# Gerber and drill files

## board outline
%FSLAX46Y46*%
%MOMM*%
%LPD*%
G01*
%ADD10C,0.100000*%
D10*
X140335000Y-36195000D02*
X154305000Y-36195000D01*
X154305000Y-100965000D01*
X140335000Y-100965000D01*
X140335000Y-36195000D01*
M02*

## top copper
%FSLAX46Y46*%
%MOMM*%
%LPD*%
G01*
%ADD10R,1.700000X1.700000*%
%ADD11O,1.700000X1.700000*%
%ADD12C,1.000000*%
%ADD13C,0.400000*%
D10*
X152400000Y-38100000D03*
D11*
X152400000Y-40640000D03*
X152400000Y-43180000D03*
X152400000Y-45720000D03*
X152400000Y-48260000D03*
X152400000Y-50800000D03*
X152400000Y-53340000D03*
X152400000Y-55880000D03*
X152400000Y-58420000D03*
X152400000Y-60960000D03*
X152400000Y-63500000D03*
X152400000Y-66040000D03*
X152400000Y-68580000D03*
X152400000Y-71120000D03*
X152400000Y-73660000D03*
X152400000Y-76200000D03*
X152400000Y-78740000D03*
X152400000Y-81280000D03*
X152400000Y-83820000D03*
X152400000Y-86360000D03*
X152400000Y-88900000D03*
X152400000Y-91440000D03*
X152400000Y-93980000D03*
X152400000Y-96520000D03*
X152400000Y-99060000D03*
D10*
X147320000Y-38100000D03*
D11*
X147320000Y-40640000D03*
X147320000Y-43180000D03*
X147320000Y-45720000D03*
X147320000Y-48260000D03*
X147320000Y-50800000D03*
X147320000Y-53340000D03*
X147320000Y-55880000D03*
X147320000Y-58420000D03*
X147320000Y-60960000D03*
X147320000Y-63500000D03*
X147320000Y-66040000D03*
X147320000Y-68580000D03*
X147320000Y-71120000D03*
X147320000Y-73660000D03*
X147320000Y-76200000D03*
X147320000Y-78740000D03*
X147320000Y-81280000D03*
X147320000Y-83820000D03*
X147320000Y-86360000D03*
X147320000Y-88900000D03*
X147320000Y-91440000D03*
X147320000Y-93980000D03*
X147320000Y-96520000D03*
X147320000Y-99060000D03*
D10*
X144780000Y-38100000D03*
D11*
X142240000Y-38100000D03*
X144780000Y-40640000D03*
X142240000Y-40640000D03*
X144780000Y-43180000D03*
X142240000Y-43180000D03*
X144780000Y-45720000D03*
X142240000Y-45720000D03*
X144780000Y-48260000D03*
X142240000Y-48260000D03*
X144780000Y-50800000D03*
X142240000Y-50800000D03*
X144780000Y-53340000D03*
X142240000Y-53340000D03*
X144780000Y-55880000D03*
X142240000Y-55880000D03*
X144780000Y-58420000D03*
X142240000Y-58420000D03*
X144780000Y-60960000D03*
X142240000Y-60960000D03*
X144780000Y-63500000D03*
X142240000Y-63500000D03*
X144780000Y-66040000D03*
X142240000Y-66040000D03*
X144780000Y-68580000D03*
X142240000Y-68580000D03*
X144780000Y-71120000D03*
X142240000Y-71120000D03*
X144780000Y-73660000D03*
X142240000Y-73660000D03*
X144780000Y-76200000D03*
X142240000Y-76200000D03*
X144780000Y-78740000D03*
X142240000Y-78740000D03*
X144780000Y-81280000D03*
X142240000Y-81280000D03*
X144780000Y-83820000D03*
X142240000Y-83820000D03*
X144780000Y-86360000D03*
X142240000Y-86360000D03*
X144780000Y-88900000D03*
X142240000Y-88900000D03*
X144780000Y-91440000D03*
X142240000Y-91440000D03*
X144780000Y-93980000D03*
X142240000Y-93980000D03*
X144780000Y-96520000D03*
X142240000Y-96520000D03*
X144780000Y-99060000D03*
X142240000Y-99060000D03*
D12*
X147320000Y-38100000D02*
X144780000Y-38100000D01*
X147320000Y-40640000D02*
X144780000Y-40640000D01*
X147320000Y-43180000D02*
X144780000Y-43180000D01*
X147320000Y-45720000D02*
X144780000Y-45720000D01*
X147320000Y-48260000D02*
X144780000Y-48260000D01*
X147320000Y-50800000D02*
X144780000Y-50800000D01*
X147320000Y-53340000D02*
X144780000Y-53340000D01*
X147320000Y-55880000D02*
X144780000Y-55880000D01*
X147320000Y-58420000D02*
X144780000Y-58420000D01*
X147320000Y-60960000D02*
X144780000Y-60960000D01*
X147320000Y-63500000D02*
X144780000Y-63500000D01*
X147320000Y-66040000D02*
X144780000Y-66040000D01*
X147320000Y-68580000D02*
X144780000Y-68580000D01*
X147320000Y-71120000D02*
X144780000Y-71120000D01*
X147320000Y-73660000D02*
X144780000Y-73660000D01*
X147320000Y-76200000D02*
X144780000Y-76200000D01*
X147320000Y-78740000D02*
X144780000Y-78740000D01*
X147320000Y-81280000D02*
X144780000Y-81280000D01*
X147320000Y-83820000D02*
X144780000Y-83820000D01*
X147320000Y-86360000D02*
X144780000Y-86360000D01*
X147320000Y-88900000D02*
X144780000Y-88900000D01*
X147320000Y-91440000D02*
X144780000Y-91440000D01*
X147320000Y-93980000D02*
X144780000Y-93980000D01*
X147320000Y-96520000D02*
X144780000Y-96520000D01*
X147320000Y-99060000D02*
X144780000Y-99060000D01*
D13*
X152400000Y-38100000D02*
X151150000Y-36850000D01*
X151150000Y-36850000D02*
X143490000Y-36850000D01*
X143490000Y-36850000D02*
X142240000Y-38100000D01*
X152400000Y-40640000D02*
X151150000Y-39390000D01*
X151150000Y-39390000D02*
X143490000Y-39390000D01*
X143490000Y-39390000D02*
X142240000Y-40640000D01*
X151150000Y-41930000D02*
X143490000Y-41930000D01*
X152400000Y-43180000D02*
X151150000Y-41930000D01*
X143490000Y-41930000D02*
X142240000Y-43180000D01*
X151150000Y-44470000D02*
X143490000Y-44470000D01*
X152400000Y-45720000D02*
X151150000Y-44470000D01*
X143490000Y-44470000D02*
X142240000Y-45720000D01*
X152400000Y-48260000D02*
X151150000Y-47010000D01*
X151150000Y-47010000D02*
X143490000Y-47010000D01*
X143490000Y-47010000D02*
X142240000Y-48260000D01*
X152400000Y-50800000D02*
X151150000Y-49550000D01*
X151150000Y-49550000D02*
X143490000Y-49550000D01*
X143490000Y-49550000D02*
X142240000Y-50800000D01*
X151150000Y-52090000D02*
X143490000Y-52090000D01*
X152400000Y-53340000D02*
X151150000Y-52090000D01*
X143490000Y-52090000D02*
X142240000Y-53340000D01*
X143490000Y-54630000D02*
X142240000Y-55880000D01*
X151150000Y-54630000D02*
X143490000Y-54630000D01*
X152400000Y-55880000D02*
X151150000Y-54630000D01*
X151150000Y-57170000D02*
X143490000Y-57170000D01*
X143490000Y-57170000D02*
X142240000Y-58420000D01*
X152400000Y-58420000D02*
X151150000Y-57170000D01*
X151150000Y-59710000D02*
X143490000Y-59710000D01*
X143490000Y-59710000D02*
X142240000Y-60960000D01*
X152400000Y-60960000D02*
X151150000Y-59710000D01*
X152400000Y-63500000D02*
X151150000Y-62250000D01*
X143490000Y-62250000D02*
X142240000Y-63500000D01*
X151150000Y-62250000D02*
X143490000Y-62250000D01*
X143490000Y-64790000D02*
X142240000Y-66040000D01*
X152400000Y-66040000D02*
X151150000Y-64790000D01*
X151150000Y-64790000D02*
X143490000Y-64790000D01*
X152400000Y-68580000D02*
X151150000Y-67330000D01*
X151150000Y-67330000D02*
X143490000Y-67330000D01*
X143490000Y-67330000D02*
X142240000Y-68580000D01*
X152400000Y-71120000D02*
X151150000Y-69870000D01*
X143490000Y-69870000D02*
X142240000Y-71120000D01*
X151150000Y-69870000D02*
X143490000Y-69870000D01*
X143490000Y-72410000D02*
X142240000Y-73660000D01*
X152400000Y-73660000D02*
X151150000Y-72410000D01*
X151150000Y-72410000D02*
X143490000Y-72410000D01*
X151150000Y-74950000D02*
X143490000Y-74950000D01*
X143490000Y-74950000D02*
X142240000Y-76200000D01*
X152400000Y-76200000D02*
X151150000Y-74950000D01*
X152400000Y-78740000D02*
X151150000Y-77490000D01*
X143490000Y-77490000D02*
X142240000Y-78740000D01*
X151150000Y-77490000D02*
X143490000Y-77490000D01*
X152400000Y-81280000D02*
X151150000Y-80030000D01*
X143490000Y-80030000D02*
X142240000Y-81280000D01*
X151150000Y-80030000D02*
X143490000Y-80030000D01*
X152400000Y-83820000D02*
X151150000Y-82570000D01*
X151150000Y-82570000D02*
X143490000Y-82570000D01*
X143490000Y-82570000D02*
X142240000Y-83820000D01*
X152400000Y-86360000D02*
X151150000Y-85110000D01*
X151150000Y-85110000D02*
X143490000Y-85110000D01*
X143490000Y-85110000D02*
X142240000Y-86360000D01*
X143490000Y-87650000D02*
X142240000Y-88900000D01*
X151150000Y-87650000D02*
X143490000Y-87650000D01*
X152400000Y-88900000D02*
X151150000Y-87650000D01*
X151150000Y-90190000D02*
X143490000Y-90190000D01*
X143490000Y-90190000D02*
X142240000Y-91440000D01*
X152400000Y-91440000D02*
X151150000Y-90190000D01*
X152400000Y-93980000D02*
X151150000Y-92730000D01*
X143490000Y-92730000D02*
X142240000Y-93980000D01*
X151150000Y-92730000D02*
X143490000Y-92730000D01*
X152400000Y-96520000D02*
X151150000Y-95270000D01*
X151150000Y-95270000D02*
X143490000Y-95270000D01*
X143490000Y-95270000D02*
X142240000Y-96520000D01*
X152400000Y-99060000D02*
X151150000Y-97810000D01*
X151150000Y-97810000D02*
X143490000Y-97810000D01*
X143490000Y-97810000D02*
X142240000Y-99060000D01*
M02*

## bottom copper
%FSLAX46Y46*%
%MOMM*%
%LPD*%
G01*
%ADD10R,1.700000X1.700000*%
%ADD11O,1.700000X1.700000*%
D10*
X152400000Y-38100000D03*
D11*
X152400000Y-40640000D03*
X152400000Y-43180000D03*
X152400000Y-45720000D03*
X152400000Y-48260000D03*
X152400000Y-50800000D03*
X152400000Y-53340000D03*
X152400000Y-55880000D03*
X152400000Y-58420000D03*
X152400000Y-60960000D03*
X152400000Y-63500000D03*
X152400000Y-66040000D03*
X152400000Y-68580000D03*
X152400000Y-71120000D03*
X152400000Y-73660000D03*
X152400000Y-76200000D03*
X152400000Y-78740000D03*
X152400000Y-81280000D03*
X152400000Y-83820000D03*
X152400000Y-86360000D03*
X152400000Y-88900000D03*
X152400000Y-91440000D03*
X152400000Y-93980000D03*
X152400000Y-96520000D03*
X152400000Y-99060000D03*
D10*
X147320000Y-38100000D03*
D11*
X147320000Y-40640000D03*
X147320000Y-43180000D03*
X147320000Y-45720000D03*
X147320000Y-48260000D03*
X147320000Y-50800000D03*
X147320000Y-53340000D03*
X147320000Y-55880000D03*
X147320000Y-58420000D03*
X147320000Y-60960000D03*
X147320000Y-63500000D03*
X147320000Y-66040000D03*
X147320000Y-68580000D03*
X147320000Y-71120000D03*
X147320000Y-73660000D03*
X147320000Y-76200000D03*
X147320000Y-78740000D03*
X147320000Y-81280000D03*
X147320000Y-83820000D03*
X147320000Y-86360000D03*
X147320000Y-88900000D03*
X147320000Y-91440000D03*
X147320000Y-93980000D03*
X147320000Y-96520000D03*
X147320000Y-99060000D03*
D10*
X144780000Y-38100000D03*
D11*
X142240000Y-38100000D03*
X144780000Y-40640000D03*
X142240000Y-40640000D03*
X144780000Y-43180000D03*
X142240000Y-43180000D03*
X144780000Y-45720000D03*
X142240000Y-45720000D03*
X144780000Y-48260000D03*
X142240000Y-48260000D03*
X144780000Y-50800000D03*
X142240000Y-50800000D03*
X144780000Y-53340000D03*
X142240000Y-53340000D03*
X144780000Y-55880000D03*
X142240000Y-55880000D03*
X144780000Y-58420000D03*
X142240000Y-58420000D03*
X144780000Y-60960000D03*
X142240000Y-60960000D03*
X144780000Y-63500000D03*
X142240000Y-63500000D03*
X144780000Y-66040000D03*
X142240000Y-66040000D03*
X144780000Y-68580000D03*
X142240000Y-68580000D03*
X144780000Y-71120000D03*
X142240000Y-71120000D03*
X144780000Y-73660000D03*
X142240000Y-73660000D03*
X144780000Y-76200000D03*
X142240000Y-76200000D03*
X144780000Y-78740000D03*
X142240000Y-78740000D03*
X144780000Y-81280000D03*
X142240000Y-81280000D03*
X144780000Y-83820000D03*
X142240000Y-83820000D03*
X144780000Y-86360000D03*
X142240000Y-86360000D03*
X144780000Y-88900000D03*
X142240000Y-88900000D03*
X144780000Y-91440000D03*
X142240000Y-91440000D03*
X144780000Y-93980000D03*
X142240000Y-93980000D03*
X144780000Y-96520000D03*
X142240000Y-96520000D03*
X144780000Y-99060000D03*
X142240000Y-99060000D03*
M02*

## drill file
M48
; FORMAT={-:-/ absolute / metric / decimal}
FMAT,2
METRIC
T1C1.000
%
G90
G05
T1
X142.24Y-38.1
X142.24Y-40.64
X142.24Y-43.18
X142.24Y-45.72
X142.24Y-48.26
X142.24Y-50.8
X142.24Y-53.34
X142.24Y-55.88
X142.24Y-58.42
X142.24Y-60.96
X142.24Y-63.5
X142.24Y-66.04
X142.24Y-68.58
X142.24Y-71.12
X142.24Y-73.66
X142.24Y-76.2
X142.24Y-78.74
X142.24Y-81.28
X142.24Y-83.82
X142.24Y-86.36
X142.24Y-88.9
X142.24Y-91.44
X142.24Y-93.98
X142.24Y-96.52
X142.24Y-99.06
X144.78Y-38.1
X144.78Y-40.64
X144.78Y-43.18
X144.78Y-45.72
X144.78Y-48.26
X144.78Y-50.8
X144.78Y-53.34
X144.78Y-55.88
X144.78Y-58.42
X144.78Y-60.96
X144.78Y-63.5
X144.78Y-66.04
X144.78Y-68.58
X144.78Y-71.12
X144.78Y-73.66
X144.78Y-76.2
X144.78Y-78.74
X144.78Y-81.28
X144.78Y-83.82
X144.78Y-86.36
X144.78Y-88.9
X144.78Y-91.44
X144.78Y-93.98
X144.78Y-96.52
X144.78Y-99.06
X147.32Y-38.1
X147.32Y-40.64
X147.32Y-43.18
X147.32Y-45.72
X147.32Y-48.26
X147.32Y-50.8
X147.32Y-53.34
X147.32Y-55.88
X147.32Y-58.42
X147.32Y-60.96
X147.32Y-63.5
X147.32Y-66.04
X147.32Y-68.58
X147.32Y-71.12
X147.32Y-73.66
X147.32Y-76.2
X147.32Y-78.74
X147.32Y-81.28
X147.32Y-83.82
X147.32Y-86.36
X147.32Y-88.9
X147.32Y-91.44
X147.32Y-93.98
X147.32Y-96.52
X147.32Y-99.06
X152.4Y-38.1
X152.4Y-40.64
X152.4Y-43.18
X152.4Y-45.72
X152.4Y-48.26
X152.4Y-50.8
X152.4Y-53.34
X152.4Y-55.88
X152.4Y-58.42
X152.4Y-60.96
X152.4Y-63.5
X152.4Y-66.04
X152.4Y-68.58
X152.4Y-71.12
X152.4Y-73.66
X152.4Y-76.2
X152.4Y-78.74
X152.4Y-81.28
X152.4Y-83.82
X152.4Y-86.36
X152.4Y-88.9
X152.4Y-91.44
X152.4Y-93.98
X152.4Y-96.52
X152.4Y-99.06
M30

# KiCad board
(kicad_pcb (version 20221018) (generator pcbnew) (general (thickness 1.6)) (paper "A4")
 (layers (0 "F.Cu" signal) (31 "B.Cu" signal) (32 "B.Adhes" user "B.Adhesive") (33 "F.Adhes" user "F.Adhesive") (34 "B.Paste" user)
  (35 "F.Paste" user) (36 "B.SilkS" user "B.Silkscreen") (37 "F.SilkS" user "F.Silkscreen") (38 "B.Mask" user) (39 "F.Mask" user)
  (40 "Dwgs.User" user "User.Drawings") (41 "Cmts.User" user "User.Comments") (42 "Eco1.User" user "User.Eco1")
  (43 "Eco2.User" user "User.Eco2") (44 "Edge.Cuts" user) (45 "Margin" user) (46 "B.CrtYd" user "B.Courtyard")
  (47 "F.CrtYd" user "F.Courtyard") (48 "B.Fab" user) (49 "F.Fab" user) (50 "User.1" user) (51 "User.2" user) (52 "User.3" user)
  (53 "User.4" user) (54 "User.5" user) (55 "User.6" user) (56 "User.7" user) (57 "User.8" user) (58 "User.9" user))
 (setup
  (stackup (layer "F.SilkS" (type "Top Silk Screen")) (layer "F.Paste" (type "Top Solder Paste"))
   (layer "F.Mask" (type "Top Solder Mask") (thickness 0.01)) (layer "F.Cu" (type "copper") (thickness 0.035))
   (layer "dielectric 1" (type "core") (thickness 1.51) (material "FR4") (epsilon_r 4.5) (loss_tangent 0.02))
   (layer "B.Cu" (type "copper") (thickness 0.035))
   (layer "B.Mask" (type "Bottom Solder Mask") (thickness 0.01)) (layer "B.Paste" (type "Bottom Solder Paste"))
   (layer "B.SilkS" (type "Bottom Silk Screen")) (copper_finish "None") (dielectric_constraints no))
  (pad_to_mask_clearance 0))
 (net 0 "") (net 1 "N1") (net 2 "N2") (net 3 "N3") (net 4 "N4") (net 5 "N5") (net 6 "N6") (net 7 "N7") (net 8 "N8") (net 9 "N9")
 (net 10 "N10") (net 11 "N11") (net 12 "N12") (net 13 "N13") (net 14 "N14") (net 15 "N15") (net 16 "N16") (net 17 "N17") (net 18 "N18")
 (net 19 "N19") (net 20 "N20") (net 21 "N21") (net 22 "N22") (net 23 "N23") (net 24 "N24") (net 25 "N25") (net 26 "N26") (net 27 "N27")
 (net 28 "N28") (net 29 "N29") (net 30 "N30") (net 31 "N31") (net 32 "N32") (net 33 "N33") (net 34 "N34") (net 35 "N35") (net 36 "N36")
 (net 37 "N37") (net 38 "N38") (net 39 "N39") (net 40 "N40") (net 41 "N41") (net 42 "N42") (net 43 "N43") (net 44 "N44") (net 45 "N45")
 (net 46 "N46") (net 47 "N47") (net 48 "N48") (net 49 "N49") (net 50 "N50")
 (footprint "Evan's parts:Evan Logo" (layer "F.Cu") (at 149.86 49.53 90)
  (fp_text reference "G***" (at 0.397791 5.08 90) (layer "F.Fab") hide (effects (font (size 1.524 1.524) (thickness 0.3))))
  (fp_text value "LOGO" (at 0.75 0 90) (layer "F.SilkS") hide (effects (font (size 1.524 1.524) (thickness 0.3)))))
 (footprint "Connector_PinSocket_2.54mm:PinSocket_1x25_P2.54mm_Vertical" (layer "F.Cu") (at 152.4 38.1)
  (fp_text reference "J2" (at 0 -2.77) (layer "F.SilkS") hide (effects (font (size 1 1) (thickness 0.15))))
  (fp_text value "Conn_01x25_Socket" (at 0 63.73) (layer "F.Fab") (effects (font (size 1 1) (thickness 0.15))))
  (pad "1" thru_hole rect (at 0 0) (size 1.7 1.7) (drill 1) (layers "*.Cu" "*.Mask") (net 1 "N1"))
  (pad "2" thru_hole oval (at 0 2.54) (size 1.7 1.7) (drill 1) (layers "*.Cu" "*.Mask") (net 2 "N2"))
  (pad "3" thru_hole oval (at 0 5.08) (size 1.7 1.7) (drill 1) (layers "*.Cu" "*.Mask") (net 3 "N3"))
  (pad "4" thru_hole oval (at 0 7.62) (size 1.7 1.7) (drill 1) (layers "*.Cu" "*.Mask") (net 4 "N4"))
  (pad "5" thru_hole oval (at 0 10.16) (size 1.7 1.7) (drill 1) (layers "*.Cu" "*.Mask") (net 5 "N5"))
  (pad "6" thru_hole oval (at 0 12.7) (size 1.7 1.7) (drill 1) (layers "*.Cu" "*.Mask") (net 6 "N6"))
  (pad "7" thru_hole oval (at 0 15.24) (size 1.7 1.7) (drill 1) (layers "*.Cu" "*.Mask") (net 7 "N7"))
  (pad "8" thru_hole oval (at 0 17.78) (size 1.7 1.7) (drill 1) (layers "*.Cu" "*.Mask") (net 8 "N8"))
  (pad "9" thru_hole oval (at 0 20.32) (size 1.7 1.7) (drill 1) (layers "*.Cu" "*.Mask") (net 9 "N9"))
  (pad "10" thru_hole oval (at 0 22.86) (size 1.7 1.7) (drill 1) (layers "*.Cu" "*.Mask") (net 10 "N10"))
  (pad "11" thru_hole oval (at 0 25.4) (size 1.7 1.7) (drill 1) (layers "*.Cu" "*.Mask") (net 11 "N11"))
  (pad "12" thru_hole oval (at 0 27.94) (size 1.7 1.7) (drill 1) (layers "*.Cu" "*.Mask") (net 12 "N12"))
  (pad "13" thru_hole oval (at 0 30.48) (size 1.7 1.7) (drill 1) (layers "*.Cu" "*.Mask") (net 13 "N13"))
  (pad "14" thru_hole oval (at 0 33.02) (size 1.7 1.7) (drill 1) (layers "*.Cu" "*.Mask") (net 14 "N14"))
  (pad "15" thru_hole oval (at 0 35.56) (size 1.7 1.7) (drill 1) (layers "*.Cu" "*.Mask") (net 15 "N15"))
  (pad "16" thru_hole oval (at 0 38.1) (size 1.7 1.7) (drill 1) (layers "*.Cu" "*.Mask") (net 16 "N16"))
  (pad "17" thru_hole oval (at 0 40.64) (size 1.7 1.7) (drill 1) (layers "*.Cu" "*.Mask") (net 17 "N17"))
  (pad "18" thru_hole oval (at 0 43.18) (size 1.7 1.7) (drill 1) (layers "*.Cu" "*.Mask") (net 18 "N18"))
  (pad "19" thru_hole oval (at 0 45.72) (size 1.7 1.7) (drill 1) (layers "*.Cu" "*.Mask") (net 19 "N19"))
  (pad "20" thru_hole oval (at 0 48.26) (size 1.7 1.7) (drill 1) (layers "*.Cu" "*.Mask") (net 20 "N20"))
  (pad "21" thru_hole oval (at 0 50.8) (size 1.7 1.7) (drill 1) (layers "*.Cu" "*.Mask") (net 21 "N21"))
  (pad "22" thru_hole oval (at 0 53.34) (size 1.7 1.7) (drill 1) (layers "*.Cu" "*.Mask") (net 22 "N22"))
  (pad "23" thru_hole oval (at 0 55.88) (size 1.7 1.7) (drill 1) (layers "*.Cu" "*.Mask") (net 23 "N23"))
  (pad "24" thru_hole oval (at 0 58.42) (size 1.7 1.7) (drill 1) (layers "*.Cu" "*.Mask") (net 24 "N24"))
  (pad "25" thru_hole oval (at 0 60.96) (size 1.7 1.7) (drill 1) (layers "*.Cu" "*.Mask") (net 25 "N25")))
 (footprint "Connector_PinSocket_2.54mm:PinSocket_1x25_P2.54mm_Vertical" (layer "F.Cu") (at 147.32 38.1)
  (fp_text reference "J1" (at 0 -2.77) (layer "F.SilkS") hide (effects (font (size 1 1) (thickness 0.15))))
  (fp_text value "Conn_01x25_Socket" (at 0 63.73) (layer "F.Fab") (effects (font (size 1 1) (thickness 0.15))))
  (pad "1" thru_hole rect (at 0 0) (size 1.7 1.7) (drill 1) (layers "*.Cu" "*.Mask") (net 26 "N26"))
  (pad "2" thru_hole oval (at 0 2.54) (size 1.7 1.7) (drill 1) (layers "*.Cu" "*.Mask") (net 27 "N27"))
  (pad "3" thru_hole oval (at 0 5.08) (size 1.7 1.7) (drill 1) (layers "*.Cu" "*.Mask") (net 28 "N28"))
  (pad "4" thru_hole oval (at 0 7.62) (size 1.7 1.7) (drill 1) (layers "*.Cu" "*.Mask") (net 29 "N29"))
  (pad "5" thru_hole oval (at 0 10.16) (size 1.7 1.7) (drill 1) (layers "*.Cu" "*.Mask") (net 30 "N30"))
  (pad "6" thru_hole oval (at 0 12.7) (size 1.7 1.7) (drill 1) (layers "*.Cu" "*.Mask") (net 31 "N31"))
  (pad "7" thru_hole oval (at 0 15.24) (size 1.7 1.7) (drill 1) (layers "*.Cu" "*.Mask") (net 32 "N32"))
  (pad "8" thru_hole oval (at 0 17.78) (size 1.7 1.7) (drill 1) (layers "*.Cu" "*.Mask") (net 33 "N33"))
  (pad "9" thru_hole oval (at 0 20.32) (size 1.7 1.7) (drill 1) (layers "*.Cu" "*.Mask") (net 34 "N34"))
  (pad "10" thru_hole oval (at 0 22.86) (size 1.7 1.7) (drill 1) (layers "*.Cu" "*.Mask") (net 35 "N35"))
  (pad "11" thru_hole oval (at 0 25.4) (size 1.7 1.7) (drill 1) (layers "*.Cu" "*.Mask") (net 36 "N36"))
  (pad "12" thru_hole oval (at 0 27.94) (size 1.7 1.7) (drill 1) (layers "*.Cu" "*.Mask") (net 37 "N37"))
  (pad "13" thru_hole oval (at 0 30.48) (size 1.7 1.7) (drill 1) (layers "*.Cu" "*.Mask") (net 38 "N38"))
  (pad "14" thru_hole oval (at 0 33.02) (size 1.7 1.7) (drill 1) (layers "*.Cu" "*.Mask") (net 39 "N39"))
  (pad "15" thru_hole oval (at 0 35.56) (size 1.7 1.7) (drill 1) (layers "*.Cu" "*.Mask") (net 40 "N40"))
  (pad "16" thru_hole oval (at 0 38.1) (size 1.7 1.7) (drill 1) (layers "*.Cu" "*.Mask") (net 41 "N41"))
  (pad "17" thru_hole oval (at 0 40.64) (size 1.7 1.7) (drill 1) (layers "*.Cu" "*.Mask") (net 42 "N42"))
  (pad "18" thru_hole oval (at 0 43.18) (size 1.7 1.7) (drill 1) (layers "*.Cu" "*.Mask") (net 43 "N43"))
  (pad "19" thru_hole oval (at 0 45.72) (size 1.7 1.7) (drill 1) (layers "*.Cu" "*.Mask") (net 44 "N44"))
  (pad "20" thru_hole oval (at 0 48.26) (size 1.7 1.7) (drill 1) (layers "*.Cu" "*.Mask") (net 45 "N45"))
  (pad "21" thru_hole oval (at 0 50.8) (size 1.7 1.7) (drill 1) (layers "*.Cu" "*.Mask") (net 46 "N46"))
  (pad "22" thru_hole oval (at 0 53.34) (size 1.7 1.7) (drill 1) (layers "*.Cu" "*.Mask") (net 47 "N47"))
  (pad "23" thru_hole oval (at 0 55.88) (size 1.7 1.7) (drill 1) (layers "*.Cu" "*.Mask") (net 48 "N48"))
  (pad "24" thru_hole oval (at 0 58.42) (size 1.7 1.7) (drill 1) (layers "*.Cu" "*.Mask") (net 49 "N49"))
  (pad "25" thru_hole oval (at 0 60.96) (size 1.7 1.7) (drill 1) (layers "*.Cu" "*.Mask") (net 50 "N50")))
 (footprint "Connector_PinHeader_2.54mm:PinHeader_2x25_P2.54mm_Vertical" (layer "B.Cu") (at 144.78 38.1 180)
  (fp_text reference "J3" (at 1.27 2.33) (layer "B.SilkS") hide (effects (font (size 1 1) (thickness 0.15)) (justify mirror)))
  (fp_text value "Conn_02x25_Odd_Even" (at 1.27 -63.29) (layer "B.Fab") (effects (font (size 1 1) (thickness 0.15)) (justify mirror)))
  (pad "1" thru_hole rect (at 0 0 180) (size 1.7 1.7) (drill 1) (layers "*.Cu" "*.Mask") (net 26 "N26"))
  (pad "2" thru_hole oval (at 2.54 0 180) (size 1.7 1.7) (drill 1) (layers "*.Cu" "*.Mask") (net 1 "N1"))
  (pad "3" thru_hole oval (at 0 -2.54 180) (size 1.7 1.7) (drill 1) (layers "*.Cu" "*.Mask") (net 27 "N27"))
  (pad "4" thru_hole oval (at 2.54 -2.54 180) (size 1.7 1.7) (drill 1) (layers "*.Cu" "*.Mask") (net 2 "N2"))
  (pad "5" thru_hole oval (at 0 -5.08 180) (size 1.7 1.7) (drill 1) (layers "*.Cu" "*.Mask") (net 28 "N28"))
  (pad "6" thru_hole oval (at 2.54 -5.08 180) (size 1.7 1.7) (drill 1) (layers "*.Cu" "*.Mask") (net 3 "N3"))
  (pad "7" thru_hole oval (at 0 -7.62 180) (size 1.7 1.7) (drill 1) (layers "*.Cu" "*.Mask") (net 29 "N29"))
  (pad "8" thru_hole oval (at 2.54 -7.62 180) (size 1.7 1.7) (drill 1) (layers "*.Cu" "*.Mask") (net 4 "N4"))
  (pad "9" thru_hole oval (at 0 -10.16 180) (size 1.7 1.7) (drill 1) (layers "*.Cu" "*.Mask") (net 30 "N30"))
  (pad "10" thru_hole oval (at 2.54 -10.16 180) (size 1.7 1.7) (drill 1) (layers "*.Cu" "*.Mask") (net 5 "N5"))
  (pad "11" thru_hole oval (at 0 -12.7 180) (size 1.7 1.7) (drill 1) (layers "*.Cu" "*.Mask") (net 31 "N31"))
  (pad "12" thru_hole oval (at 2.54 -12.7 180) (size 1.7 1.7) (drill 1) (layers "*.Cu" "*.Mask") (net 6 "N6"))
  (pad "13" thru_hole oval (at 0 -15.24 180) (size 1.7 1.7) (drill 1) (layers "*.Cu" "*.Mask") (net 32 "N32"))
  (pad "14" thru_hole oval (at 2.54 -15.24 180) (size 1.7 1.7) (drill 1) (layers "*.Cu" "*.Mask") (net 7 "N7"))
  (pad "15" thru_hole oval (at 0 -17.78 180) (size 1.7 1.7) (drill 1) (layers "*.Cu" "*.Mask") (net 33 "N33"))
  (pad "16" thru_hole oval (at 2.54 -17.78 180) (size 1.7 1.7) (drill 1) (layers "*.Cu" "*.Mask") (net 8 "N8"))
  (pad "17" thru_hole oval (at 0 -20.32 180) (size 1.7 1.7) (drill 1) (layers "*.Cu" "*.Mask") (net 34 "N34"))
  (pad "18" thru_hole oval (at 2.54 -20.32 180) (size 1.7 1.7) (drill 1) (layers "*.Cu" "*.Mask") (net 9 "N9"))
  (pad "19" thru_hole oval (at 0 -22.86 180) (size 1.7 1.7) (drill 1) (layers "*.Cu" "*.Mask") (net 35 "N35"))
  (pad "20" thru_hole oval (at 2.54 -22.86 180) (size 1.7 1.7) (drill 1) (layers "*.Cu" "*.Mask") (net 10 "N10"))
  (pad "21" thru_hole oval (at 0 -25.4 180) (size 1.7 1.7) (drill 1) (layers "*.Cu" "*.Mask") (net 36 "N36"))
  (pad "22" thru_hole oval (at 2.54 -25.4 180) (size 1.7 1.7) (drill 1) (layers "*.Cu" "*.Mask") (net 11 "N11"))
  (pad "23" thru_hole oval (at 0 -27.94 180) (size 1.7 1.7) (drill 1) (layers "*.Cu" "*.Mask") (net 37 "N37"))
  (pad "24" thru_hole oval (at 2.54 -27.94 180) (size 1.7 1.7) (drill 1) (layers "*.Cu" "*.Mask") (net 12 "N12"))
  (pad "25" thru_hole oval (at 0 -30.48 180) (size 1.7 1.7) (drill 1) (layers "*.Cu" "*.Mask") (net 38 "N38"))
  (pad "26" thru_hole oval (at 2.54 -30.48 180) (size 1.7 1.7) (drill 1) (layers "*.Cu" "*.Mask") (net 13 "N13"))
  (pad "27" thru_hole oval (at 0 -33.02 180) (size 1.7 1.7) (drill 1) (layers "*.Cu" "*.Mask") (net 39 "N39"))
  (pad "28" thru_hole oval (at 2.54 -33.02 180) (size 1.7 1.7) (drill 1) (layers "*.Cu" "*.Mask") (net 14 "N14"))
  (pad "29" thru_hole oval (at 0 -35.56 180) (size 1.7 1.7) (drill 1) (layers "*.Cu" "*.Mask") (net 40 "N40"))
  (pad "30" thru_hole oval (at 2.54 -35.56 180) (size 1.7 1.7) (drill 1) (layers "*.Cu" "*.Mask") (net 15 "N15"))
  (pad "31" thru_hole oval (at 0 -38.1 180) (size 1.7 1.7) (drill 1) (layers "*.Cu" "*.Mask") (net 41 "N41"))
  (pad "32" thru_hole oval (at 2.54 -38.1 180) (size 1.7 1.7) (drill 1) (layers "*.Cu" "*.Mask") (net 16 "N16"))
  (pad "33" thru_hole oval (at 0 -40.64 180) (size 1.7 1.7) (drill 1) (layers "*.Cu" "*.Mask") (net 42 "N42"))
  (pad "34" thru_hole oval (at 2.54 -40.64 180) (size 1.7 1.7) (drill 1) (layers "*.Cu" "*.Mask") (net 17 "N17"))
  (pad "35" thru_hole oval (at 0 -43.18 180) (size 1.7 1.7) (drill 1) (layers "*.Cu" "*.Mask") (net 43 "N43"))
  (pad "36" thru_hole oval (at 2.54 -43.18 180) (size 1.7 1.7) (drill 1) (layers "*.Cu" "*.Mask") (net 18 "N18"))
  (pad "37" thru_hole oval (at 0 -45.72 180) (size 1.7 1.7) (drill 1) (layers "*.Cu" "*.Mask") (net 44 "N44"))
  (pad "38" thru_hole oval (at 2.54 -45.72 180) (size 1.7 1.7) (drill 1) (layers "*.Cu" "*.Mask") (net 19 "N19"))
  (pad "39" thru_hole oval (at 0 -48.26 180) (size 1.7 1.7) (drill 1) (layers "*.Cu" "*.Mask") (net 45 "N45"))
  (pad "40" thru_hole oval (at 2.54 -48.26 180) (size 1.7 1.7) (drill 1) (layers "*.Cu" "*.Mask") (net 20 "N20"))
  (pad "41" thru_hole oval (at 0 -50.8 180) (size 1.7 1.7) (drill 1) (layers "*.Cu" "*.Mask") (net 46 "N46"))
  (pad "42" thru_hole oval (at 2.54 -50.8 180) (size 1.7 1.7) (drill 1) (layers "*.Cu" "*.Mask") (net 21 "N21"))
  (pad "43" thru_hole oval (at 0 -53.34 180) (size 1.7 1.7) (drill 1) (layers "*.Cu" "*.Mask") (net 47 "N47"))
  (pad "44" thru_hole oval (at 2.54 -53.34 180) (size 1.7 1.7) (drill 1) (layers "*.Cu" "*.Mask") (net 22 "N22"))
  (pad "45" thru_hole oval (at 0 -55.88 180) (size 1.7 1.7) (drill 1) (layers "*.Cu" "*.Mask") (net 48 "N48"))
  (pad "46" thru_hole oval (at 2.54 -55.88 180) (size 1.7 1.7) (drill 1) (layers "*.Cu" "*.Mask") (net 23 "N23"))
  (pad "47" thru_hole oval (at 0 -58.42 180) (size 1.7 1.7) (drill 1) (layers "*.Cu" "*.Mask") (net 49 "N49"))
  (pad "48" thru_hole oval (at 2.54 -58.42 180) (size 1.7 1.7) (drill 1) (layers "*.Cu" "*.Mask") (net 24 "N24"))
  (pad "49" thru_hole oval (at 0 -60.96 180) (size 1.7 1.7) (drill 1) (layers "*.Cu" "*.Mask") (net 50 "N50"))
  (pad "50" thru_hole oval (at 2.54 -60.96 180) (size 1.7 1.7) (drill 1) (layers "*.Cu" "*.Mask") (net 25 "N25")))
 (gr_rect (start 140.335 36.195) (end 154.305 100.965) (stroke (width 0.1) (type default)) (fill none) (layer "Edge.Cuts"))
 (segment (start 147.32 38.1) (end 144.78 38.1) (width 1) (layer "F.Cu") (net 26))
 (segment (start 147.32 40.64) (end 144.78 40.64) (width 1) (layer "F.Cu") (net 27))
 (segment (start 147.32 43.18) (end 144.78 43.18) (width 1) (layer "F.Cu") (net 28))
 (segment (start 147.32 45.72) (end 144.78 45.72) (width 1) (layer "F.Cu") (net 29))
 (segment (start 147.32 48.26) (end 144.78 48.26) (width 1) (layer "F.Cu") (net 30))
 (segment (start 147.32 50.8) (end 144.78 50.8) (width 1) (layer "F.Cu") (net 31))
 (segment (start 147.32 53.34) (end 144.78 53.34) (width 1) (layer "F.Cu") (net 32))
 (segment (start 147.32 55.88) (end 144.78 55.88) (width 1) (layer "F.Cu") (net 33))
 (segment (start 147.32 58.42) (end 144.78 58.42) (width 1) (layer "F.Cu") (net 34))
 (segment (start 147.32 60.96) (end 144.78 60.96) (width 1) (layer "F.Cu") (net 35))
 (segment (start 147.32 63.5) (end 144.78 63.5) (width 1) (layer "F.Cu") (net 36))
 (segment (start 147.32 66.04) (end 144.78 66.04) (width 1) (layer "F.Cu") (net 37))
 (segment (start 147.32 68.58) (end 144.78 68.58) (width 1) (layer "F.Cu") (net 38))
 (segment (start 147.32 71.12) (end 144.78 71.12) (width 1) (layer "F.Cu") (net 39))
 (segment (start 147.32 73.66) (end 144.78 73.66) (width 1) (layer "F.Cu") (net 40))
 (segment (start 147.32 76.2) (end 144.78 76.2) (width 1) (layer "F.Cu") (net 41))
 (segment (start 147.32 78.74) (end 144.78 78.74) (width 1) (layer "F.Cu") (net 42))
 (segment (start 147.32 81.28) (end 144.78 81.28) (width 1) (layer "F.Cu") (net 43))
 (segment (start 147.32 83.82) (end 144.78 83.82) (width 1) (layer "F.Cu") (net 44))
 (segment (start 147.32 86.36) (end 144.78 86.36) (width 1) (layer "F.Cu") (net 45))
 (segment (start 147.32 88.9) (end 144.78 88.9) (width 1) (layer "F.Cu") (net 46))
 (segment (start 147.32 91.44) (end 144.78 91.44) (width 1) (layer "F.Cu") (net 47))
 (segment (start 147.32 93.98) (end 144.78 93.98) (width 1) (layer "F.Cu") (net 48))
 (segment (start 147.32 96.52) (end 144.78 96.52) (width 1) (layer "F.Cu") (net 49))
 (segment (start 147.32 99.06) (end 144.78 99.06) (width 1) (layer "F.Cu") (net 50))
 (segment (start 152.4 38.1) (end 151.15 36.85) (width 0.4) (layer "F.Cu") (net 1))
 (segment (start 151.15 36.85) (end 143.49 36.85) (width 0.4) (layer "F.Cu") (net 1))
 (segment (start 143.49 36.85) (end 142.24 38.1) (width 0.4) (layer "F.Cu") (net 1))
 (segment (start 152.4 40.64) (end 151.15 39.39) (width 0.4) (layer "F.Cu") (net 2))
 (segment (start 151.15 39.39) (end 143.49 39.39) (width 0.4) (layer "F.Cu") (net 2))
 (segment (start 143.49 39.39) (end 142.24 40.64) (width 0.4) (layer "F.Cu") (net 2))
 (segment (start 151.15 41.93) (end 143.49 41.93) (width 0.4) (layer "F.Cu") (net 3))
 (segment (start 152.4 43.18) (end 151.15 41.93) (width 0.4) (layer "F.Cu") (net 3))
 (segment (start 143.49 41.93) (end 142.24 43.18) (width 0.4) (layer "F.Cu") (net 3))
 (segment (start 151.15 44.47) (end 143.49 44.47) (width 0.4) (layer "F.Cu") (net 4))
 (segment (start 152.4 45.72) (end 151.15 44.47) (width 0.4) (layer "F.Cu") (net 4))
 (segment (start 143.49 44.47) (end 142.24 45.72) (width 0.4) (layer "F.Cu") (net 4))
 (segment (start 152.4 48.26) (end 151.15 47.01) (width 0.4) (layer "F.Cu") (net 5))
 (segment (start 151.15 47.01) (end 143.49 47.01) (width 0.4) (layer "F.Cu") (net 5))
 (segment (start 143.49 47.01) (end 142.24 48.26) (width 0.4) (layer "F.Cu") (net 5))
 (segment (start 152.4 50.8) (end 151.15 49.55) (width 0.4) (layer "F.Cu") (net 6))
 (segment (start 151.15 49.55) (end 143.49 49.55) (width 0.4) (layer "F.Cu") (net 6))
 (segment (start 143.49 49.55) (end 142.24 50.8) (width 0.4) (layer "F.Cu") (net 6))
 (segment (start 151.15 52.09) (end 143.49 52.09) (width 0.4) (layer "F.Cu") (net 7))
 (segment (start 152.4 53.34) (end 151.15 52.09) (width 0.4) (layer "F.Cu") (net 7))
 (segment (start 143.49 52.09) (end 142.24 53.34) (width 0.4) (layer "F.Cu") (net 7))
 (segment (start 143.49 54.63) (end 142.24 55.88) (width 0.4) (layer "F.Cu") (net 8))
 (segment (start 151.15 54.63) (end 143.49 54.63) (width 0.4) (layer "F.Cu") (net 8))
 (segment (start 152.4 55.88) (end 151.15 54.63) (width 0.4) (layer "F.Cu") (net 8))
 (segment (start 151.15 57.17) (end 143.49 57.17) (width 0.4) (layer "F.Cu") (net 9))
 (segment (start 143.49 57.17) (end 142.24 58.42) (width 0.4) (layer "F.Cu") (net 9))
 (segment (start 152.4 58.42) (end 151.15 57.17) (width 0.4) (layer "F.Cu") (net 9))
 (segment (start 151.15 59.71) (end 143.49 59.71) (width 0.4) (layer "F.Cu") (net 10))
 (segment (start 143.49 59.71) (end 142.24 60.96) (width 0.4) (layer "F.Cu") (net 10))
 (segment (start 152.4 60.96) (end 151.15 59.71) (width 0.4) (layer "F.Cu") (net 10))
 (segment (start 152.4 63.5) (end 151.15 62.25) (width 0.4) (layer "F.Cu") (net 11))
 (segment (start 143.49 62.25) (end 142.24 63.5) (width 0.4) (layer "F.Cu") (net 11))
 (segment (start 151.15 62.25) (end 143.49 62.25) (width 0.4) (layer "F.Cu") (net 11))
 (segment (start 143.49 64.79) (end 142.24 66.04) (width 0.4) (layer "F.Cu") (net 12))
 (segment (start 152.4 66.04) (end 151.15 64.79) (width 0.4) (layer "F.Cu") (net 12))
 (segment (start 151.15 64.79) (end 143.49 64.79) (width 0.4) (layer "F.Cu") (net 12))
 (segment (start 152.4 68.58) (end 151.15 67.33) (width 0.4) (layer "F.Cu") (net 13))
 (segment (start 151.15 67.33) (end 143.49 67.33) (width 0.4) (layer "F.Cu") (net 13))
 (segment (start 143.49 67.33) (end 142.24 68.58) (width 0.4) (layer "F.Cu") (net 13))
 (segment (start 152.4 71.12) (end 151.15 69.87) (width 0.4) (layer "F.Cu") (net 14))
 (segment (start 143.49 69.87) (end 142.24 71.12) (width 0.4) (layer "F.Cu") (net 14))
 (segment (start 151.15 69.87) (end 143.49 69.87) (width 0.4) (layer "F.Cu") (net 14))
 (segment (start 143.49 72.41) (end 142.24 73.66) (width 0.4) (layer "F.Cu") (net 15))
 (segment (start 152.4 73.66) (end 151.15 72.41) (width 0.4) (layer "F.Cu") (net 15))
 (segment (start 151.15 72.41) (end 143.49 72.41) (width 0.4) (layer "F.Cu") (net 15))
 (segment (start 151.15 74.95) (end 143.49 74.95) (width 0.4) (layer "F.Cu") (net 16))
 (segment (start 143.49 74.95) (end 142.24 76.2) (width 0.4) (layer "F.Cu") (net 16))
 (segment (start 152.4 76.2) (end 151.15 74.95) (width 0.4) (layer "F.Cu") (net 16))
 (segment (start 152.4 78.74) (end 151.15 77.49) (width 0.4) (layer "F.Cu") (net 17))
 (segment (start 143.49 77.49) (end 142.24 78.74) (width 0.4) (layer "F.Cu") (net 17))
 (segment (start 151.15 77.49) (end 143.49 77.49) (width 0.4) (layer "F.Cu") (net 17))
 (segment (start 152.4 81.28) (end 151.15 80.03) (width 0.4) (layer "F.Cu") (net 18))
 (segment (start 143.49 80.03) (end 142.24 81.28) (width 0.4) (layer "F.Cu") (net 18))
 (segment (start 151.15 80.03) (end 143.49 80.03) (width 0.4) (layer "F.Cu") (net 18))
 (segment (start 152.4 83.82) (end 151.15 82.57) (width 0.4) (layer "F.Cu") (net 19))
 (segment (start 151.15 82.57) (end 143.49 82.57) (width 0.4) (layer "F.Cu") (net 19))
 (segment (start 143.49 82.57) (end 142.24 83.82) (width 0.4) (layer "F.Cu") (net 19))
 (segment (start 152.4 86.36) (end 151.15 85.11) (width 0.4) (layer "F.Cu") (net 20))
 (segment (start 151.15 85.11) (end 143.49 85.11) (width 0.4) (layer "F.Cu") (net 20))
 (segment (start 143.49 85.11) (end 142.24 86.36) (width 0.4) (layer "F.Cu") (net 20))
 (segment (start 143.49 87.65) (end 142.24 88.9) (width 0.4) (layer "F.Cu") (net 21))
 (segment (start 151.15 87.65) (end 143.49 87.65) (width 0.4) (layer "F.Cu") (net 21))
 (segment (start 152.4 88.9) (end 151.15 87.65) (width 0.4) (layer "F.Cu") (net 21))
 (segment (start 151.15 90.19) (end 143.49 90.19) (width 0.4) (layer "F.Cu") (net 22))
 (segment (start 143.49 90.19) (end 142.24 91.44) (width 0.4) (layer "F.Cu") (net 22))
 (segment (start 152.4 91.44) (end 151.15 90.19) (width 0.4) (layer "F.Cu") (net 22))
 (segment (start 152.4 93.98) (end 151.15 92.73) (width 0.4) (layer "F.Cu") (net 23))
 (segment (start 143.49 92.73) (end 142.24 93.98) (width 0.4) (layer "F.Cu") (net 23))
 (segment (start 151.15 92.73) (end 143.49 92.73) (width 0.4) (layer "F.Cu") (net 23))
 (segment (start 152.4 96.52) (end 151.15 95.27) (width 0.4) (layer "F.Cu") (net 24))
 (segment (start 151.15 95.27) (end 143.49 95.27) (width 0.4) (layer "F.Cu") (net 24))
 (segment (start 143.49 95.27) (end 142.24 96.52) (width 0.4) (layer "F.Cu") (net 24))
 (segment (start 152.4 99.06) (end 151.15 97.81) (width 0.4) (layer "F.Cu") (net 25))
 (segment (start 151.15 97.81) (end 143.49 97.81) (width 0.4) (layer "F.Cu") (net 25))
 (segment (start 143.49 97.81) (end 142.24 99.06) (width 0.4) (layer "F.Cu") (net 25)))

